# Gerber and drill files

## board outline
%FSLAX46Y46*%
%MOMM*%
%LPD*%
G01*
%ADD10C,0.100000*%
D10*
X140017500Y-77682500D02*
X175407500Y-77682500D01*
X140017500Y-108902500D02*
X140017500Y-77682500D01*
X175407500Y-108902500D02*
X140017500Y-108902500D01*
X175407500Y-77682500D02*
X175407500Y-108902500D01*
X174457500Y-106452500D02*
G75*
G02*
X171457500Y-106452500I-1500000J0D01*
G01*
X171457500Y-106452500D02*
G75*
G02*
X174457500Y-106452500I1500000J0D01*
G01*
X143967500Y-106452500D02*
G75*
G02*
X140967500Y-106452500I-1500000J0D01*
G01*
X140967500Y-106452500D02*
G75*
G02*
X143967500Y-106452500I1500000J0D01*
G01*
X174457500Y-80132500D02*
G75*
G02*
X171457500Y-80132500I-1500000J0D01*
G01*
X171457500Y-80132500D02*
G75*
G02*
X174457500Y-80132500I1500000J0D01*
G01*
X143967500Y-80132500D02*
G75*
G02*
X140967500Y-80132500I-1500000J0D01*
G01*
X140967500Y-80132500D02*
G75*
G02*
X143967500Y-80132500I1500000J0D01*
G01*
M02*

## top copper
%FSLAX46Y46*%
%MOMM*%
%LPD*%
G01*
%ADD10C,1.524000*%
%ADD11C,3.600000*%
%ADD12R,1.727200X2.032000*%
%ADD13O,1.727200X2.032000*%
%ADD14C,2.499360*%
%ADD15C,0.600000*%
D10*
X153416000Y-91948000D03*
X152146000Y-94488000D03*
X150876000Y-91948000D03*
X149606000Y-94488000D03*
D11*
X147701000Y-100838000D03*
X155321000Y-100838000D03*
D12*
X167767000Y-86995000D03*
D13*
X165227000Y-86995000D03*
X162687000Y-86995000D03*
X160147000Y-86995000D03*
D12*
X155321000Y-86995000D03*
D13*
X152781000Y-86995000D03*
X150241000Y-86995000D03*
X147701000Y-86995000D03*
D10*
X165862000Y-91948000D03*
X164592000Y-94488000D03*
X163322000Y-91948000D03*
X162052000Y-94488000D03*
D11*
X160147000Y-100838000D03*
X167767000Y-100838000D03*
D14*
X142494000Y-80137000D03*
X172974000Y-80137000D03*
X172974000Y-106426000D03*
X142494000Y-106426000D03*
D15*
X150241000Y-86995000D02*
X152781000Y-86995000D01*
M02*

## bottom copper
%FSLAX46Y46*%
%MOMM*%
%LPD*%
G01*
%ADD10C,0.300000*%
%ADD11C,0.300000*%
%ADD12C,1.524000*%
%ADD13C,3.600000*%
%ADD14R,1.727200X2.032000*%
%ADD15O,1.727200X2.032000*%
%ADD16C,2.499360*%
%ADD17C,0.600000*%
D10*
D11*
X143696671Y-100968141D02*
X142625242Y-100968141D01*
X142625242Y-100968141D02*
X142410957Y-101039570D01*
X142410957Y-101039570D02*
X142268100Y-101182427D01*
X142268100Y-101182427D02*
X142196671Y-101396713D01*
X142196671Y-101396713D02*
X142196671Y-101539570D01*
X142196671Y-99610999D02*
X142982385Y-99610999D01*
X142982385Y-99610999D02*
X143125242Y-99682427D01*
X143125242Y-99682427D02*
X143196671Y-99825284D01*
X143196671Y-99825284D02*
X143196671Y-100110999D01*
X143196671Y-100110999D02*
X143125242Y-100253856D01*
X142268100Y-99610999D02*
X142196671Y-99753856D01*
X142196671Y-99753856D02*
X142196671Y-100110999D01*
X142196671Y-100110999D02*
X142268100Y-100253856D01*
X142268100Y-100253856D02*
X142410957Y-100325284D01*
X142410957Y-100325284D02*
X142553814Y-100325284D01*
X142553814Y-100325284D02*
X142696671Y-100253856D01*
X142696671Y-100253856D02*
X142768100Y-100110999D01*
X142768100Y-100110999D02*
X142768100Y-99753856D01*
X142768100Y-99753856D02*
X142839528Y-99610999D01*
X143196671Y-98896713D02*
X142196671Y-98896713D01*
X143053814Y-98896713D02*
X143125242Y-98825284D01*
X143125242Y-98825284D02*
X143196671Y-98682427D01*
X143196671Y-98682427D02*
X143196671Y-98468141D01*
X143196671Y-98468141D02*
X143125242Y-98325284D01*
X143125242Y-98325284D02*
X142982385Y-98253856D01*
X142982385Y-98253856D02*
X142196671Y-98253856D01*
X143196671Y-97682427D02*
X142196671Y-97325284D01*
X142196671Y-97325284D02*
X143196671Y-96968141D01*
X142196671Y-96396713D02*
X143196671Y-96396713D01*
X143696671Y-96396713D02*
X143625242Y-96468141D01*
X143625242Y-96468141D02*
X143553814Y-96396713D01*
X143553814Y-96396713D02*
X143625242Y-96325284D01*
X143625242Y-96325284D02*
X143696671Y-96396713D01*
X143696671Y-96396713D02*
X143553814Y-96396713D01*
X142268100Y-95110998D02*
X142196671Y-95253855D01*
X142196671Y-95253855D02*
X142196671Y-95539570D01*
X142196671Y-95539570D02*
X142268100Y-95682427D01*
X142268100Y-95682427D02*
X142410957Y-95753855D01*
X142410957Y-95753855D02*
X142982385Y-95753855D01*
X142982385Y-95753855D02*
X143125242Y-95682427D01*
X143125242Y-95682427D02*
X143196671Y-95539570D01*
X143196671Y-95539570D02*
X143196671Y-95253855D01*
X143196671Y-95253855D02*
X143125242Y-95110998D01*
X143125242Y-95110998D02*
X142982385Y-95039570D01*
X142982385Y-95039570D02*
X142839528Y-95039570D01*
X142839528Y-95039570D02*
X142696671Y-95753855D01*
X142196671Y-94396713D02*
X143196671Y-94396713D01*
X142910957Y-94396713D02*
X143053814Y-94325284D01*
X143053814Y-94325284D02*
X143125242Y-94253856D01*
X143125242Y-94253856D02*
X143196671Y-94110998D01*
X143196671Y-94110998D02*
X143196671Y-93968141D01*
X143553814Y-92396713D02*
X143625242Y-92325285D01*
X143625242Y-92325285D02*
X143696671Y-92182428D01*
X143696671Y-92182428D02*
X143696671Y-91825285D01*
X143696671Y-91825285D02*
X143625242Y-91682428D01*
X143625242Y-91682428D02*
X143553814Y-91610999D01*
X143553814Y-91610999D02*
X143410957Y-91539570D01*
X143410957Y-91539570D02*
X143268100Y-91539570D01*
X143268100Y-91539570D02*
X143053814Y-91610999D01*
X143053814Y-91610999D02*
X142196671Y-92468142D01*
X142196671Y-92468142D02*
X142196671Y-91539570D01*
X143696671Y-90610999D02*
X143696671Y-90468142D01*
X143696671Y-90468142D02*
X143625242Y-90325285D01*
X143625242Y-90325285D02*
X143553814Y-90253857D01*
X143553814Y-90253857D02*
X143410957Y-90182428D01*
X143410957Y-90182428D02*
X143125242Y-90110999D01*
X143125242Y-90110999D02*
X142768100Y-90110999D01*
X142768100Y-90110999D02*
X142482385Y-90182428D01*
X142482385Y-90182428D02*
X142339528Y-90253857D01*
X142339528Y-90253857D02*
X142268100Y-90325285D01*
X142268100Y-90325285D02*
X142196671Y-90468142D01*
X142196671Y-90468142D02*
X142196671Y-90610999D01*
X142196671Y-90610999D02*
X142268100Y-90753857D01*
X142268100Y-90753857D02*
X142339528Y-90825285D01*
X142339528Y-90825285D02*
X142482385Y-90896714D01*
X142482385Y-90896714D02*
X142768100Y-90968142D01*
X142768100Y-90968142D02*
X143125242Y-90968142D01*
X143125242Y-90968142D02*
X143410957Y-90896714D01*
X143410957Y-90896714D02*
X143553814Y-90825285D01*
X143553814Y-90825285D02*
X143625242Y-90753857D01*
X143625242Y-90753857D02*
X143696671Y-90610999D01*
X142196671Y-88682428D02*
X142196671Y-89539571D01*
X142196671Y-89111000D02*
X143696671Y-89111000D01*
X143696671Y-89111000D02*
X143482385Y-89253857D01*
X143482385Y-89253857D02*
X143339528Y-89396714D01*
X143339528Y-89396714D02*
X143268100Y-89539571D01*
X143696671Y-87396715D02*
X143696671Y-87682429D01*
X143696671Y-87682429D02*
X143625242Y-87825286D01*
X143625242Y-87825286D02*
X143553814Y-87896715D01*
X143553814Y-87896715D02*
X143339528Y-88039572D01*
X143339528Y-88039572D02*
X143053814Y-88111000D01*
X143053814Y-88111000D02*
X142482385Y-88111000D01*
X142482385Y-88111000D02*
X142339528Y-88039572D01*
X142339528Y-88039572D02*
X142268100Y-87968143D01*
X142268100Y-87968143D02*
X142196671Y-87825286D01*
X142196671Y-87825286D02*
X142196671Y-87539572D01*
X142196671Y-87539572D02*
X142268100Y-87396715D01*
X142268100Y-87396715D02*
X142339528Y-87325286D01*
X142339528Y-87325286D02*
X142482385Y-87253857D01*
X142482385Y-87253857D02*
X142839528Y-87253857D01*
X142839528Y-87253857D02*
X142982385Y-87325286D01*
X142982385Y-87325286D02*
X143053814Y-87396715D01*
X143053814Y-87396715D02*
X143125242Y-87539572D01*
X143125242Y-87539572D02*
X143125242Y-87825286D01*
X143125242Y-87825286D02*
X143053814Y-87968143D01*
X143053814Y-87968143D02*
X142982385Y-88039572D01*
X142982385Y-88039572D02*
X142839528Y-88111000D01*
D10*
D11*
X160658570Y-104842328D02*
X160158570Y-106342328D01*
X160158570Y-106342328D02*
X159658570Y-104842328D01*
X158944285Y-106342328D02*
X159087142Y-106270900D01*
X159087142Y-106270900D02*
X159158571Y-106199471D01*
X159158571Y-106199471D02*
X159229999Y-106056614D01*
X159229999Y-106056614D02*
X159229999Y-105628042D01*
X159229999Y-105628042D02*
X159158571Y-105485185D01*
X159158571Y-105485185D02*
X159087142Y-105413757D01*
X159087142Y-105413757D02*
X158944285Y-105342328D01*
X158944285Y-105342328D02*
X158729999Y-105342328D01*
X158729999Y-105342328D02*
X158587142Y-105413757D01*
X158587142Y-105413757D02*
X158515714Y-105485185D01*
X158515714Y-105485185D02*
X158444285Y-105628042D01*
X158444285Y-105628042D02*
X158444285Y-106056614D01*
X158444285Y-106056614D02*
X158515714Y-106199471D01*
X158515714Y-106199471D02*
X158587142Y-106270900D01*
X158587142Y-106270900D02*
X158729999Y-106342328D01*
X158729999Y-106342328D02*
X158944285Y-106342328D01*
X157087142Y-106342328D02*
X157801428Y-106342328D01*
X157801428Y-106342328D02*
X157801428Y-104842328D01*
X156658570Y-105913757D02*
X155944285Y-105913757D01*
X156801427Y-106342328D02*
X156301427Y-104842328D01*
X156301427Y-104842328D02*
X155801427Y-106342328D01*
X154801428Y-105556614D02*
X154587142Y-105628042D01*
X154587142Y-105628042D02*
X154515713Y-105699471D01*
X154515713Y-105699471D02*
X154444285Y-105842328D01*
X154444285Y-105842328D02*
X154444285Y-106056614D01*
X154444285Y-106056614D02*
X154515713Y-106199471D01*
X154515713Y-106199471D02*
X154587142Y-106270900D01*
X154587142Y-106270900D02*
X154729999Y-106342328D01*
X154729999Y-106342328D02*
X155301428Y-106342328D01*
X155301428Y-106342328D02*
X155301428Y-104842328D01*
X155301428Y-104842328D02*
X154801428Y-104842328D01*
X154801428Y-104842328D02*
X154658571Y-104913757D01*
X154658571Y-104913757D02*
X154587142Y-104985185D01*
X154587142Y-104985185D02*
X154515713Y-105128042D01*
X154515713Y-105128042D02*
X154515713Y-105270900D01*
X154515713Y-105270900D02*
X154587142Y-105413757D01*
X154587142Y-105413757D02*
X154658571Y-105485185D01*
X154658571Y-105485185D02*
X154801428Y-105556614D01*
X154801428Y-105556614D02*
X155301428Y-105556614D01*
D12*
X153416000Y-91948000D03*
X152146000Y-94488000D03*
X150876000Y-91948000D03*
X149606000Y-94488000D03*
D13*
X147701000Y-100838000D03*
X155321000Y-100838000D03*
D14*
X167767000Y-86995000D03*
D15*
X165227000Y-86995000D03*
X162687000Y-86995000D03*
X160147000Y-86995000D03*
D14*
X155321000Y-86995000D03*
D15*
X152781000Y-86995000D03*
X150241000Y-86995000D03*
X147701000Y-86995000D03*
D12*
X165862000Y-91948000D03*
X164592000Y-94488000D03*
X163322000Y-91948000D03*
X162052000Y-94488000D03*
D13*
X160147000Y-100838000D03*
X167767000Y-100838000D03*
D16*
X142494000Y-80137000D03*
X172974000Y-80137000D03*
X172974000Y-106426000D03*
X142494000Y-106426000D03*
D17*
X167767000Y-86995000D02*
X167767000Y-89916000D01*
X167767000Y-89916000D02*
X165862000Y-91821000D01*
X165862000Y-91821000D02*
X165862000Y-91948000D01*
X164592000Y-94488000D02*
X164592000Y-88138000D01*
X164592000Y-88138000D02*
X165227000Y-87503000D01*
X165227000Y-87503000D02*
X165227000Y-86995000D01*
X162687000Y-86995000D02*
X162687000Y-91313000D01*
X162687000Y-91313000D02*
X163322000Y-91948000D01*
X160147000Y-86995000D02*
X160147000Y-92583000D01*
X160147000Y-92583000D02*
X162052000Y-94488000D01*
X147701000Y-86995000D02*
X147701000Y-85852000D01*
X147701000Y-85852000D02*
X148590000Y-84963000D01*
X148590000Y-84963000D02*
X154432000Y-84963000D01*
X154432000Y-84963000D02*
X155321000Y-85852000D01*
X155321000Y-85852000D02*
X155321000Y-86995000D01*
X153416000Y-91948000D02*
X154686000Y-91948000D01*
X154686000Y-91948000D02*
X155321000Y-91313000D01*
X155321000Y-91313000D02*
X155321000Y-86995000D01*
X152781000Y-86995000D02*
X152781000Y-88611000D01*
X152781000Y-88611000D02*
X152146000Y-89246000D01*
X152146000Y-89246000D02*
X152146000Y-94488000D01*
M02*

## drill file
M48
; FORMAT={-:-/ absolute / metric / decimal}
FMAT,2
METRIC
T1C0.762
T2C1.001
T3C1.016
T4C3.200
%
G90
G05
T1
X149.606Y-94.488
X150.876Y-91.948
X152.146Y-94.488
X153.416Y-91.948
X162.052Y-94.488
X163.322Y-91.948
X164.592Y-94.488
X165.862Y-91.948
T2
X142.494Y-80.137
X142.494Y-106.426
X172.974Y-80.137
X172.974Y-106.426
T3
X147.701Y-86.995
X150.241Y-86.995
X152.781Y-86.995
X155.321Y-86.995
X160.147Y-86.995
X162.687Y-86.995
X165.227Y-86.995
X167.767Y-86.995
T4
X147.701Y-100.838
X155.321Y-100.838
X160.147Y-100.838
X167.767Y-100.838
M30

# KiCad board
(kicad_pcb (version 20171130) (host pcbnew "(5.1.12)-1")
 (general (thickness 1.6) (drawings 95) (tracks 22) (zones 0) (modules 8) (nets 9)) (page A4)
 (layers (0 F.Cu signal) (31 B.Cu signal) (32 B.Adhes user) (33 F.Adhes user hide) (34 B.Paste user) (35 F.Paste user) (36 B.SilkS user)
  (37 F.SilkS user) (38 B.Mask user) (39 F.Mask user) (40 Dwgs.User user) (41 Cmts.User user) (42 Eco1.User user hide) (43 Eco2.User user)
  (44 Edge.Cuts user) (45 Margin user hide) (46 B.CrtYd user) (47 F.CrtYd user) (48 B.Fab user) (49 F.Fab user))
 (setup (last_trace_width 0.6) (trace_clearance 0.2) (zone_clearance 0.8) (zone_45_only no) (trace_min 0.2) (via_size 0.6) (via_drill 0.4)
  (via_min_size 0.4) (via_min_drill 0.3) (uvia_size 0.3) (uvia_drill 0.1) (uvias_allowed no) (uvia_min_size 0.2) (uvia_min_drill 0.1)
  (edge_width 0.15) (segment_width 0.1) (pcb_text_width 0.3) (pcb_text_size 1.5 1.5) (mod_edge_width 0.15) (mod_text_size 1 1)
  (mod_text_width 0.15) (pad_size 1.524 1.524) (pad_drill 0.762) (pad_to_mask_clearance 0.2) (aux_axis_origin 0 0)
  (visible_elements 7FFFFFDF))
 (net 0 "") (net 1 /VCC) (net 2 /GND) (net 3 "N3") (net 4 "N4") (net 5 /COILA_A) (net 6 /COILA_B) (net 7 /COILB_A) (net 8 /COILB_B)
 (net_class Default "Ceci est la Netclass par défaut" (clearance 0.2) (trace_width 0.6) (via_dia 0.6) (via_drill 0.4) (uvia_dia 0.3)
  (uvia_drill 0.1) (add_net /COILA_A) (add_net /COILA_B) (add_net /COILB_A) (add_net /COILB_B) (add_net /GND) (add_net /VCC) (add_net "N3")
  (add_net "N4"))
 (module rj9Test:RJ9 (layer F.Cu) (at 151.511 100.838)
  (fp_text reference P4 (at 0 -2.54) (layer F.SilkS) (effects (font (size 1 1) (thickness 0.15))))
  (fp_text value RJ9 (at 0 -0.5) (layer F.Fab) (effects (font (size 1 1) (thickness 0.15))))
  (pad 1 thru_hole circle (at 1.905 -8.89) (size 1.524 1.524) (drill 0.762) (layers *.Cu *.Mask F.SilkS) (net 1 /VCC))
  (pad 2 thru_hole circle (at 0.635 -6.35) (size 1.524 1.524) (drill 0.762) (layers *.Cu *.Mask F.SilkS) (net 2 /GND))
  (pad 3 thru_hole circle (at -0.635 -8.89) (size 1.524 1.524) (drill 0.762) (layers *.Cu *.Mask F.SilkS) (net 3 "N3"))
  (pad 4 thru_hole circle (at -1.905 -6.35) (size 1.524 1.524) (drill 0.762) (layers *.Cu *.Mask F.SilkS) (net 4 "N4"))
  (pad "" thru_hole circle (at -3.81 0) (size 3.6 3.6) (drill 3.2) (layers *.Cu *.Mask F.SilkS))
  (pad "" thru_hole circle (at 3.81 0) (size 3.6 3.6) (drill 3.2) (layers *.Cu *.Mask F.SilkS)))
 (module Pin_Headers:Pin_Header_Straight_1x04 (layer F.Cu) (at 167.767 86.995 270)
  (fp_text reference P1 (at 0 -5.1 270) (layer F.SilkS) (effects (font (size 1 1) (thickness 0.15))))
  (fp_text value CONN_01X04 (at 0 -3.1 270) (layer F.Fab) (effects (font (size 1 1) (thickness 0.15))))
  (pad 1 thru_hole rect (at 0 0 270) (size 2.032 1.7272) (drill 1.016) (layers *.Cu *.Mask F.SilkS) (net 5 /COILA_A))
  (pad 2 thru_hole oval (at 0 2.54 270) (size 2.032 1.7272) (drill 1.016) (layers *.Cu *.Mask F.SilkS) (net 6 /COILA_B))
  (pad 3 thru_hole oval (at 0 5.08 270) (size 2.032 1.7272) (drill 1.016) (layers *.Cu *.Mask F.SilkS) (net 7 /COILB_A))
  (pad 4 thru_hole oval (at 0 7.62 270) (size 2.032 1.7272) (drill 1.016) (layers *.Cu *.Mask F.SilkS) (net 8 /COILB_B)))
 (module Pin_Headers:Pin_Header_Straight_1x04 (layer F.Cu) (at 155.321 86.995 270)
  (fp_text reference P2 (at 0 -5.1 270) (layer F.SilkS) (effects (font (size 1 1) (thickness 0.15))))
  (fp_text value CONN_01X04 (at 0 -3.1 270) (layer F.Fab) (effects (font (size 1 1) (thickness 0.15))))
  (pad 1 thru_hole rect (at 0 0 270) (size 2.032 1.7272) (drill 1.016) (layers *.Cu *.Mask F.SilkS) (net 1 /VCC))
  (pad 2 thru_hole oval (at 0 2.54 270) (size 2.032 1.7272) (drill 1.016) (layers *.Cu *.Mask F.SilkS) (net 2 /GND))
  (pad 3 thru_hole oval (at 0 5.08 270) (size 2.032 1.7272) (drill 1.016) (layers *.Cu *.Mask F.SilkS) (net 2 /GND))
  (pad 4 thru_hole oval (at 0 7.62 270) (size 2.032 1.7272) (drill 1.016) (layers *.Cu *.Mask F.SilkS) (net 1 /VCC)))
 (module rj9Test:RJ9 (layer F.Cu) (at 163.957 100.838)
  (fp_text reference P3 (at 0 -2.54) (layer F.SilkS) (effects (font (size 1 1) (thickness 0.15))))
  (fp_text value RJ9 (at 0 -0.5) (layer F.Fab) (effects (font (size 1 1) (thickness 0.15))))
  (pad 1 thru_hole circle (at 1.905 -8.89) (size 1.524 1.524) (drill 0.762) (layers *.Cu *.Mask F.SilkS) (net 5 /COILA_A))
  (pad 2 thru_hole circle (at 0.635 -6.35) (size 1.524 1.524) (drill 0.762) (layers *.Cu *.Mask F.SilkS) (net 6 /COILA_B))
  (pad 3 thru_hole circle (at -0.635 -8.89) (size 1.524 1.524) (drill 0.762) (layers *.Cu *.Mask F.SilkS) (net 7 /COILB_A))
  (pad 4 thru_hole circle (at -1.905 -6.35) (size 1.524 1.524) (drill 0.762) (layers *.Cu *.Mask F.SilkS) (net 8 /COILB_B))
  (pad "" thru_hole circle (at -3.81 0) (size 3.6 3.6) (drill 3.2) (layers *.Cu *.Mask F.SilkS))
  (pad "" thru_hole circle (at 3.81 0) (size 3.6 3.6) (drill 3.2) (layers *.Cu *.Mask F.SilkS)))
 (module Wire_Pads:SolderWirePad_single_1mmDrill (layer F.Cu) (at 142.494 80.137)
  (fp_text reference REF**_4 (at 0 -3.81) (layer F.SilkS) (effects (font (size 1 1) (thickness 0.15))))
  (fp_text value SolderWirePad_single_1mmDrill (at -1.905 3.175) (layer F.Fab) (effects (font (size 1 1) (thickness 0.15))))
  (pad 1 thru_hole circle (at 0 0) (size 2.49936 2.49936) (drill 1.00076) (layers *.Cu *.Mask F.SilkS)))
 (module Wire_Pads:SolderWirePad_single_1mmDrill (layer F.Cu) (at 172.974 80.137)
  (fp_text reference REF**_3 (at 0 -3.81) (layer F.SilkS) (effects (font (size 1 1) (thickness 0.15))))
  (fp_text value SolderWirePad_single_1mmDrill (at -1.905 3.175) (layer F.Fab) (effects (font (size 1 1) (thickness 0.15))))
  (pad 1 thru_hole circle (at 0 0) (size 2.49936 2.49936) (drill 1.00076) (layers *.Cu *.Mask F.SilkS)))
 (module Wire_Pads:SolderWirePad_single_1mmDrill (layer F.Cu) (at 172.974 106.426)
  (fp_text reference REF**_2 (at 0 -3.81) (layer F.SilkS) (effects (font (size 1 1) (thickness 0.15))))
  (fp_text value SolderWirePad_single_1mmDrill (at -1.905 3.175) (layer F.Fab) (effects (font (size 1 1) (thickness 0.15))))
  (pad 1 thru_hole circle (at 0 0) (size 2.49936 2.49936) (drill 1.00076) (layers *.Cu *.Mask F.SilkS)))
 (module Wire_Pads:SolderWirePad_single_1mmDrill (layer F.Cu) (at 142.494 106.426)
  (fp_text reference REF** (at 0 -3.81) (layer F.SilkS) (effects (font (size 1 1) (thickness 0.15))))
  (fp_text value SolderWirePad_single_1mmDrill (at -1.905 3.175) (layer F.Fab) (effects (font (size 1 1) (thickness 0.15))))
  (pad 1 thru_hole circle (at 0 0) (size 2.49936 2.49936) (drill 1.00076) (layers *.Cu *.Mask F.SilkS)))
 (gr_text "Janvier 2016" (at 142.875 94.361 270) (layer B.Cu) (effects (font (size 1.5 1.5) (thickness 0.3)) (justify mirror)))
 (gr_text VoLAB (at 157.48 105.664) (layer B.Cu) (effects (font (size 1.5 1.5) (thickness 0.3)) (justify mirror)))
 (gr_line (start 140.0175 77.6825) (end 175.4075 77.6825) (layer Edge.Cuts) (width 0.1))
 (gr_line (start 140.0175 108.9025) (end 140.0175 77.6825) (layer Edge.Cuts) (width 0.1))
 (gr_line (start 175.4075 108.9025) (end 140.0175 108.9025) (layer Edge.Cuts) (width 0.1))
 (gr_line (start 175.4075 77.6825) (end 175.4075 108.9025) (layer Edge.Cuts) (width 0.1))
 (gr_circle (center 172.9575 106.4525) (end 172.9575 104.9525) (layer Edge.Cuts) (width 0.1))
 (gr_circle (center 142.4675 106.4525) (end 142.4675 104.9525) (layer Edge.Cuts) (width 0.1))
 (gr_circle (center 172.9575 80.1325) (end 172.9575 78.6325) (layer Edge.Cuts) (width 0.1))
 (gr_circle (center 142.4675 80.1325) (end 142.4675 78.6325) (layer Edge.Cuts) (width 0.1))
 (segment (start 167.767 86.995) (end 167.767 89.916) (width 0.6) (layer B.Cu) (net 5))
 (segment (start 167.767 89.916) (end 165.862 91.821) (width 0.6) (layer B.Cu) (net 5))
 (segment (start 165.862 91.821) (end 165.862 91.948) (width 0.6) (layer B.Cu) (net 5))
 (segment (start 164.592 94.488) (end 164.592 88.138) (width 0.6) (layer B.Cu) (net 6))
 (segment (start 164.592 88.138) (end 165.227 87.503) (width 0.6) (layer B.Cu) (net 6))
 (segment (start 165.227 87.503) (end 165.227 86.995) (width 0.6) (layer B.Cu) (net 6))
 (segment (start 162.687 86.995) (end 162.687 91.313) (width 0.6) (layer B.Cu) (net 7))
 (segment (start 162.687 91.313) (end 163.322 91.948) (width 0.6) (layer B.Cu) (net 7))
 (segment (start 160.147 86.995) (end 160.147 92.583) (width 0.6) (layer B.Cu) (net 8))
 (segment (start 160.147 92.583) (end 162.052 94.488) (width 0.6) (layer B.Cu) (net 8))
 (segment (start 147.701 86.995) (end 147.701 85.852) (width 0.6) (layer B.Cu) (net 1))
 (segment (start 147.701 85.852) (end 148.59 84.963) (width 0.6) (layer B.Cu) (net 1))
 (segment (start 148.59 84.963) (end 154.432 84.963) (width 0.6) (layer B.Cu) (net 1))
 (segment (start 154.432 84.963) (end 155.321 85.852) (width 0.6) (layer B.Cu) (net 1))
 (segment (start 155.321 85.852) (end 155.321 86.995) (width 0.6) (layer B.Cu) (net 1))
 (segment (start 153.416 91.948) (end 154.686 91.948) (width 0.6) (layer B.Cu) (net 1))
 (segment (start 154.686 91.948) (end 155.321 91.313) (width 0.6) (layer B.Cu) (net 1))
 (segment (start 155.321 91.313) (end 155.321 86.995) (width 0.6) (layer B.Cu) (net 1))
 (segment (start 152.781 86.995) (end 152.781 88.611) (width 0.6) (layer B.Cu) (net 2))
 (segment (start 152.781 88.611) (end 152.146 89.246) (width 0.6) (layer B.Cu) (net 2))
 (segment (start 152.146 89.246) (end 152.146 94.488) (width 0.6) (layer B.Cu) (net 2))
 (segment (start 150.241 86.995) (end 152.781 86.995) (width 0.6) (layer F.Cu) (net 2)))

